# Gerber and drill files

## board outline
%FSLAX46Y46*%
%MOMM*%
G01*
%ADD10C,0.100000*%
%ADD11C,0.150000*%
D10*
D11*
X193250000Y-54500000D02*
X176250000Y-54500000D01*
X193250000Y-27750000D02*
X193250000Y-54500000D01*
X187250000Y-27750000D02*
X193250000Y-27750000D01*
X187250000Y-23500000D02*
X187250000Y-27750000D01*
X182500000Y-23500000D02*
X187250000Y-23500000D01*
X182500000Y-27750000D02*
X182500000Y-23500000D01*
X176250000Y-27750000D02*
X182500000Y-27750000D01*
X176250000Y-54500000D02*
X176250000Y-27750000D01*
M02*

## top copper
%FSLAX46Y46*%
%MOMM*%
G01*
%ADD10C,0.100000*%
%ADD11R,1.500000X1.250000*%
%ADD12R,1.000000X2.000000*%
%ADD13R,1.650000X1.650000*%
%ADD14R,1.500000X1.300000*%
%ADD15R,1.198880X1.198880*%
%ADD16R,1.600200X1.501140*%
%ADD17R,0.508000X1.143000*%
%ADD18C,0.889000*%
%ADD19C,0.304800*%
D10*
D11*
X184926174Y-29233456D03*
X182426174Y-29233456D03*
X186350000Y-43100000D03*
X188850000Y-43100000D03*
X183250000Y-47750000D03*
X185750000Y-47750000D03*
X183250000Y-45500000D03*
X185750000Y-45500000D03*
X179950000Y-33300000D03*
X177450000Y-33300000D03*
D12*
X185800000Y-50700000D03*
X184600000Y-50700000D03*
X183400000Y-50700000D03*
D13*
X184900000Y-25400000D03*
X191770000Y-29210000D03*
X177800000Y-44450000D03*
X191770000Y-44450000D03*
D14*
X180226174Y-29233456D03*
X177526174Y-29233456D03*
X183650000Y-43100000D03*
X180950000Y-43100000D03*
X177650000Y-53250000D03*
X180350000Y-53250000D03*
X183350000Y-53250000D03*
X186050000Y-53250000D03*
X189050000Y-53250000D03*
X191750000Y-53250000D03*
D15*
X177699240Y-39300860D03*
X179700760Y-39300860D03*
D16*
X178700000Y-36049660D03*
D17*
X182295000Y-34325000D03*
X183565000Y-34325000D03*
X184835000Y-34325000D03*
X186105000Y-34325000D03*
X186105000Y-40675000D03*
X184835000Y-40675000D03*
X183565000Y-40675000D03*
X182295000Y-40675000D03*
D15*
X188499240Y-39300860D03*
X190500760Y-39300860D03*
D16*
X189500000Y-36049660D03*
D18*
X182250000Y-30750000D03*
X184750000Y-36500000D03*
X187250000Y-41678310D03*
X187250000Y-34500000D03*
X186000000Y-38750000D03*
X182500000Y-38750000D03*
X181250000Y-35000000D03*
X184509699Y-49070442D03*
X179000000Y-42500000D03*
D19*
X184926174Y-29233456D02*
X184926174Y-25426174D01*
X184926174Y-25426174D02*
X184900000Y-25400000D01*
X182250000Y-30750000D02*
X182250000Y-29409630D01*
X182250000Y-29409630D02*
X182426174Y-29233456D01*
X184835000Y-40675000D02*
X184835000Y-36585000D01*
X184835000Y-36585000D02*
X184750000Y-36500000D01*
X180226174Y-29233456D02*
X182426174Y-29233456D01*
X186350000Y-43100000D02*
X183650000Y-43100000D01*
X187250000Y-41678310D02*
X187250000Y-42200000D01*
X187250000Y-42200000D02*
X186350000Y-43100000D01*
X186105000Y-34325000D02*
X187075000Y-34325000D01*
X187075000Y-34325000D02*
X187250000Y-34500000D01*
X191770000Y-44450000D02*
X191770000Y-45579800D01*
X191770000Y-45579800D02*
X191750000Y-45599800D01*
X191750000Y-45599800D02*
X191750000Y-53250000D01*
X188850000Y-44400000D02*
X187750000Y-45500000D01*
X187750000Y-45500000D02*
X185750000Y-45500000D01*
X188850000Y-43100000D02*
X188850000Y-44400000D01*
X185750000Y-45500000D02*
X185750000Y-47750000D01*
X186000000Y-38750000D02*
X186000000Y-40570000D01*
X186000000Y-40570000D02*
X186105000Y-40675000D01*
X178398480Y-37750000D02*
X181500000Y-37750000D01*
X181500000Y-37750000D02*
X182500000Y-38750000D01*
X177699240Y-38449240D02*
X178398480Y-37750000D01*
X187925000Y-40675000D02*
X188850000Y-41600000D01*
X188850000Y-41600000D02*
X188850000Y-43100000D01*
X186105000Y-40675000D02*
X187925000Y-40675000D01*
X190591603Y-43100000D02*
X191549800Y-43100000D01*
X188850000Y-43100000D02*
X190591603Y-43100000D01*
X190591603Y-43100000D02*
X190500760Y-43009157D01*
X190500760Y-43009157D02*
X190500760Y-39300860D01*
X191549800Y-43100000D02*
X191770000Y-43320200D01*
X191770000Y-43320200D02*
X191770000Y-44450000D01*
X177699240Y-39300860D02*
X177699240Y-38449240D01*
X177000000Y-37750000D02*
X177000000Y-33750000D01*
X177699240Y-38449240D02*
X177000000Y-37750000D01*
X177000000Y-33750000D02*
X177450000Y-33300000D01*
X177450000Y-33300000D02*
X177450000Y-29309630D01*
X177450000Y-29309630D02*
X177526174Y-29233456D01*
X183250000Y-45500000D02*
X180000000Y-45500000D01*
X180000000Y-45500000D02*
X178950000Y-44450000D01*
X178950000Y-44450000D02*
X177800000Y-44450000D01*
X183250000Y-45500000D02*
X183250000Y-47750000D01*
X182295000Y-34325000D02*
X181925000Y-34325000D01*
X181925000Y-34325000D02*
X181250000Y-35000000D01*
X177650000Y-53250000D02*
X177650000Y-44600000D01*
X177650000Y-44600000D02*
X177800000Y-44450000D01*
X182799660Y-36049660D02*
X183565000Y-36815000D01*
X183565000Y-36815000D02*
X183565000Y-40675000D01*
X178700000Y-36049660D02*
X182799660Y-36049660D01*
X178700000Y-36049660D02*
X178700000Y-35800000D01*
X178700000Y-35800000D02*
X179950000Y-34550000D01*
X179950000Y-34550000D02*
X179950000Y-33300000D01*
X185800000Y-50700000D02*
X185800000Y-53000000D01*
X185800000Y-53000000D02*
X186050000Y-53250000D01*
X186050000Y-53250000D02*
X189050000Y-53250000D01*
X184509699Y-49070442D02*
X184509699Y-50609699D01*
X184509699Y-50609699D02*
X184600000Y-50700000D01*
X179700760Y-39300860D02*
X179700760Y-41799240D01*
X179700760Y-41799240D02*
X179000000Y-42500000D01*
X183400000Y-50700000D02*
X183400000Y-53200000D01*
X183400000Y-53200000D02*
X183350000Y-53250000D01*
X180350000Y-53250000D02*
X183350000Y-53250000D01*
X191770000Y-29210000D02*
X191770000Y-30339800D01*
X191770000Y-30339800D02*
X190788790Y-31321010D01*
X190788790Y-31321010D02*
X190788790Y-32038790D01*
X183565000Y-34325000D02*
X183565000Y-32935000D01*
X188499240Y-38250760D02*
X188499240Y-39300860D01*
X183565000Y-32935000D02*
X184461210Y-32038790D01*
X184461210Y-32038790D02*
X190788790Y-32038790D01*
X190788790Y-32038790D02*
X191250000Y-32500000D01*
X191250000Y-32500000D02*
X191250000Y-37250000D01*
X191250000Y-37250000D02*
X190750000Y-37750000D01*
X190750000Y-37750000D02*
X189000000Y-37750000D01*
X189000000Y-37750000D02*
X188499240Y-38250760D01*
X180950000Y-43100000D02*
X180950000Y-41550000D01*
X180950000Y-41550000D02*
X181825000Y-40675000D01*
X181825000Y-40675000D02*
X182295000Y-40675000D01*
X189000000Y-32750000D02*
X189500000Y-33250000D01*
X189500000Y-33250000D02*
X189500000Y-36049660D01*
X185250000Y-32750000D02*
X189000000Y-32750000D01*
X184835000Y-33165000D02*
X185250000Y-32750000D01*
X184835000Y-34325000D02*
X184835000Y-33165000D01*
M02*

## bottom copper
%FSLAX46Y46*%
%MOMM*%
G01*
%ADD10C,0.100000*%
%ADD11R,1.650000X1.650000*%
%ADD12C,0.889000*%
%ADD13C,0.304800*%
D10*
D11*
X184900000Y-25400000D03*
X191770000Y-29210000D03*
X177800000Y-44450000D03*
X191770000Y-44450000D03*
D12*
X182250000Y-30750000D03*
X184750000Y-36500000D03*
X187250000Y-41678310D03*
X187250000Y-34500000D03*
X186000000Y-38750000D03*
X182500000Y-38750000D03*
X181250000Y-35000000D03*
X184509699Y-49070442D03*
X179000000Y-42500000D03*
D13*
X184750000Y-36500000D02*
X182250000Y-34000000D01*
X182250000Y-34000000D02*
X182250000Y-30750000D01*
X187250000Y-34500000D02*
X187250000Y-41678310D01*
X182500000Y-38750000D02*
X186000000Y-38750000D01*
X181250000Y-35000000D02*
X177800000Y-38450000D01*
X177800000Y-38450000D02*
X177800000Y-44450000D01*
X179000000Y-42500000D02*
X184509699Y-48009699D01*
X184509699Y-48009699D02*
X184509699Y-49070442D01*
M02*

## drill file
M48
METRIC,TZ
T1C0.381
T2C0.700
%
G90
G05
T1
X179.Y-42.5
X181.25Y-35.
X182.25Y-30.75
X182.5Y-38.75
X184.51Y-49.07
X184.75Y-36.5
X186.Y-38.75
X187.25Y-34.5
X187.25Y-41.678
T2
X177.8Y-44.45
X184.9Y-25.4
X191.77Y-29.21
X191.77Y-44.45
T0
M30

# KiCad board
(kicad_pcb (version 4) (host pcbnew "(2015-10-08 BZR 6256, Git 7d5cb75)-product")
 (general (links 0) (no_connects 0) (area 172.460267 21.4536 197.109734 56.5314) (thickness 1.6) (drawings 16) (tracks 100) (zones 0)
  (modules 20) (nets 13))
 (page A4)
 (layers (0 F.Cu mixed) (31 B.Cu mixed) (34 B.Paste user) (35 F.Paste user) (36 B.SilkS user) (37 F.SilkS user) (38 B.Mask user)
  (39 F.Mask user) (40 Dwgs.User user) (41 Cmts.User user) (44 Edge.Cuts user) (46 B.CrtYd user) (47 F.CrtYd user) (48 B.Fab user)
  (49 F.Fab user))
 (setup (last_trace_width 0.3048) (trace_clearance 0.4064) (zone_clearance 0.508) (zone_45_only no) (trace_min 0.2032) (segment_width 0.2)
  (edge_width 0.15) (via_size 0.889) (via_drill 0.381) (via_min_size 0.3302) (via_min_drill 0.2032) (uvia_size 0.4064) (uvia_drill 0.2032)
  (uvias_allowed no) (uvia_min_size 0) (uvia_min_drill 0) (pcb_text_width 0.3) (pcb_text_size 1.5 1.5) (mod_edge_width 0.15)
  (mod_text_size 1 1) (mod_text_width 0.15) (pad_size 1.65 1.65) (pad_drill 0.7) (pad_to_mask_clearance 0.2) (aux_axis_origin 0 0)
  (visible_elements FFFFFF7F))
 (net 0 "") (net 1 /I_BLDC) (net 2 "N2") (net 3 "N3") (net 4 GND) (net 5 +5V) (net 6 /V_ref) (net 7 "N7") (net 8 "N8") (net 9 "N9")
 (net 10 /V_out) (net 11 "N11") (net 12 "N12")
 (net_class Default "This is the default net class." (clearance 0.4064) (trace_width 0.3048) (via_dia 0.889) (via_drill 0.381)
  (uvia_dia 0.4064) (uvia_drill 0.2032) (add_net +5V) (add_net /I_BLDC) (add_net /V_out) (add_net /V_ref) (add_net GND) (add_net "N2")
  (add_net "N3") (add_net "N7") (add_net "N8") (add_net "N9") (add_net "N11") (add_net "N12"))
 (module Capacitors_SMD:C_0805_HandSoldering (layer F.Cu) (at 183.676174 29.233456 180)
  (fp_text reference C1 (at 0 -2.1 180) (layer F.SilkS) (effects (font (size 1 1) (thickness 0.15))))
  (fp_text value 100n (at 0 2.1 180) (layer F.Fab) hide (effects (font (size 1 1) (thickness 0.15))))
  (pad 1 smd rect (at -1.25 0 180) (size 1.5 1.25) (layers F.Cu F.Paste F.Mask) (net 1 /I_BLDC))
  (pad 2 smd rect (at 1.25 0 180) (size 1.5 1.25) (layers F.Cu F.Paste F.Mask) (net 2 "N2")))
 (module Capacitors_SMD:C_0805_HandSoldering (layer F.Cu) (at 187.6 43.1)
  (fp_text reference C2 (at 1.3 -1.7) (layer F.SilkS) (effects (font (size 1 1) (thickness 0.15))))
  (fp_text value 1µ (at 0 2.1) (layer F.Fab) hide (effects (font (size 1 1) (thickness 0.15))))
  (pad 1 smd rect (at -1.25 0) (size 1.5 1.25) (layers F.Cu F.Paste F.Mask) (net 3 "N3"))
  (pad 2 smd rect (at 1.25 0) (size 1.5 1.25) (layers F.Cu F.Paste F.Mask) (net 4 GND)))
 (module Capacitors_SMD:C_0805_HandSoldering (layer F.Cu) (at 184.5 47.75)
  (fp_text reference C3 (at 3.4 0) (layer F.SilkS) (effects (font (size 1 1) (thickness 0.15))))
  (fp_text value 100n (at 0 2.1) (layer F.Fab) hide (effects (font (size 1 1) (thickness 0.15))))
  (pad 1 smd rect (at -1.25 0) (size 1.5 1.25) (layers F.Cu F.Paste F.Mask) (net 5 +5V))
  (pad 2 smd rect (at 1.25 0) (size 1.5 1.25) (layers F.Cu F.Paste F.Mask) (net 4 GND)))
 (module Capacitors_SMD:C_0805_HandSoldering (layer F.Cu) (at 184.5 45.5)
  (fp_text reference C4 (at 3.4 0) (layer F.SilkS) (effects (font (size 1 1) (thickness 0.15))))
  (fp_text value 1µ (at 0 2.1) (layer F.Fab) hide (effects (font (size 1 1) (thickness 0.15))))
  (pad 1 smd rect (at -1.25 0) (size 1.5 1.25) (layers F.Cu F.Paste F.Mask) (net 5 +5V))
  (pad 2 smd rect (at 1.25 0) (size 1.5 1.25) (layers F.Cu F.Paste F.Mask) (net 4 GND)))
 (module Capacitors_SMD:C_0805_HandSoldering (layer F.Cu) (at 178.7 33.3 180)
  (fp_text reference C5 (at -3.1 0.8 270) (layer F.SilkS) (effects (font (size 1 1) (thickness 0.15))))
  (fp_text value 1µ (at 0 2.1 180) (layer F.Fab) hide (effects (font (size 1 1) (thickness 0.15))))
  (pad 1 smd rect (at -1.25 0 180) (size 1.5 1.25) (layers F.Cu F.Paste F.Mask) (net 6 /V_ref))
  (pad 2 smd rect (at 1.25 0 180) (size 1.5 1.25) (layers F.Cu F.Paste F.Mask) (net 4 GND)))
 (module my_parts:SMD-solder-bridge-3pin (layer F.Cu) (at 184.6 50.7 180) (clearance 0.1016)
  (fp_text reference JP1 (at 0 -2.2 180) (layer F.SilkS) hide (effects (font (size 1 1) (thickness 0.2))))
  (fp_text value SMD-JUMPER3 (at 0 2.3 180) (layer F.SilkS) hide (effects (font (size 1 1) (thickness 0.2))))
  (pad 1 smd rect (at -1.2 0 180) (size 1 2) (layers F.Cu F.Mask) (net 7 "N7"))
  (pad 2 smd rect (at 0 0 180) (size 1 2) (layers F.Cu F.Mask) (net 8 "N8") (solder_mask_margin 0.3))
  (pad 3 smd rect (at 1.2 0 180) (size 1 2) (layers F.Cu F.Mask) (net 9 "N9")))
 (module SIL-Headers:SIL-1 (layer F.Cu) (at 184.9 25.4)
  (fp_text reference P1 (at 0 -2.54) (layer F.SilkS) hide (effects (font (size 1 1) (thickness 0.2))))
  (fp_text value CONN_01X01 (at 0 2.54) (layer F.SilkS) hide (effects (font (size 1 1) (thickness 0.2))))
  (pad 1 thru_hole rect (at 0 0) (size 1.65 1.65) (drill 0.7) (layers *.Cu *.Mask) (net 1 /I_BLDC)))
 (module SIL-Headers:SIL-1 (layer F.Cu) (at 191.77 29.21)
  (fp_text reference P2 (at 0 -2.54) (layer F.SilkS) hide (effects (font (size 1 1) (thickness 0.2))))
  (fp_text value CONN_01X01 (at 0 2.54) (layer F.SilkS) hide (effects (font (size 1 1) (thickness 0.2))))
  (pad 1 thru_hole rect (at 0 0) (size 1.65 1.65) (drill 0.7) (layers *.Cu *.Mask) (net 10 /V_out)))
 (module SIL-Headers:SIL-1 (layer F.Cu) (at 177.8 44.45)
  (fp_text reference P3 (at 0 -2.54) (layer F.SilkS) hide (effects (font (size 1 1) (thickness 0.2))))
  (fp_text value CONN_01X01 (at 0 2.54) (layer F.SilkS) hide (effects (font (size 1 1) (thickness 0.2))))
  (pad 1 thru_hole rect (at 0 0) (size 1.65 1.65) (drill 0.7) (layers *.Cu *.Mask) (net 5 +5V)))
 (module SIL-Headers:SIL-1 (layer F.Cu) (at 191.77 44.45)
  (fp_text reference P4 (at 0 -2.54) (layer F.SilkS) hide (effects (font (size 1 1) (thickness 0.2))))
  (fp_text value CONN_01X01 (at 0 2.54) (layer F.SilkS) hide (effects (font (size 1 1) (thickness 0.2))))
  (pad 1 thru_hole rect (at 0 0) (size 1.65 1.65) (drill 0.7) (layers *.Cu *.Mask) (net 4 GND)))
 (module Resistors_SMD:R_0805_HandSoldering (layer F.Cu) (at 178.876174 29.233456 180)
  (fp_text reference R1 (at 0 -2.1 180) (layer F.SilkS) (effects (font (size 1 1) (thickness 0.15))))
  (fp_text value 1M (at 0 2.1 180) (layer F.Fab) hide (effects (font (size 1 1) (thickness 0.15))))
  (pad 1 smd rect (at -1.35 0 180) (size 1.5 1.3) (layers F.Cu F.Paste F.Mask) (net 2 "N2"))
  (pad 2 smd rect (at 1.35 0 180) (size 1.5 1.3) (layers F.Cu F.Paste F.Mask) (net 4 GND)))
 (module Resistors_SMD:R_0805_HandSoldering (layer F.Cu) (at 182.3 43.1 180)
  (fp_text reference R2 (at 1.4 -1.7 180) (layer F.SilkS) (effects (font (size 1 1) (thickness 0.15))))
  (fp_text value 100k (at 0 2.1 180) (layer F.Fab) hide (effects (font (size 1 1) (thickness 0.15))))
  (pad 1 smd rect (at -1.35 0 180) (size 1.5 1.3) (layers F.Cu F.Paste F.Mask) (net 3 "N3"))
  (pad 2 smd rect (at 1.35 0 180) (size 1.5 1.3) (layers F.Cu F.Paste F.Mask) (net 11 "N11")))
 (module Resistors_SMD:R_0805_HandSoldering (layer F.Cu) (at 179 53.25)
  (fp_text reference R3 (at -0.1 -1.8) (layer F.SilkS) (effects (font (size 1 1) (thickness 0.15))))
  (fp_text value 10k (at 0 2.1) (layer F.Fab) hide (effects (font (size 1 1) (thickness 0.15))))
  (pad 1 smd rect (at -1.35 0) (size 1.5 1.3) (layers F.Cu F.Paste F.Mask) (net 5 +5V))
  (pad 2 smd rect (at 1.35 0) (size 1.5 1.3) (layers F.Cu F.Paste F.Mask) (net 9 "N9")))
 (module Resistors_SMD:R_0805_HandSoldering (layer F.Cu) (at 184.7 53.25)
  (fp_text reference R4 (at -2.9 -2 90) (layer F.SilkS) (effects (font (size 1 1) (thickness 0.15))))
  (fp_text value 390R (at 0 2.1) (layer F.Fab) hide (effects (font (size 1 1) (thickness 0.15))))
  (pad 1 smd rect (at -1.35 0) (size 1.5 1.3) (layers F.Cu F.Paste F.Mask) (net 9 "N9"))
  (pad 2 smd rect (at 1.35 0) (size 1.5 1.3) (layers F.Cu F.Paste F.Mask) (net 7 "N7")))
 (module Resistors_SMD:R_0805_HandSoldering (layer F.Cu) (at 190.4 53.25)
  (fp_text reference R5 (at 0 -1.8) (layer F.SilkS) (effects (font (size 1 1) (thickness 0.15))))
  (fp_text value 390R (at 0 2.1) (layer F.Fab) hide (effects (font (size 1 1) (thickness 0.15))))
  (pad 1 smd rect (at -1.35 0) (size 1.5 1.3) (layers F.Cu F.Paste F.Mask) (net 7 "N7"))
  (pad 2 smd rect (at 1.35 0) (size 1.5 1.3) (layers F.Cu F.Paste F.Mask) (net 4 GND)))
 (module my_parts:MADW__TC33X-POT (layer F.Cu) (at 178.7 37.5)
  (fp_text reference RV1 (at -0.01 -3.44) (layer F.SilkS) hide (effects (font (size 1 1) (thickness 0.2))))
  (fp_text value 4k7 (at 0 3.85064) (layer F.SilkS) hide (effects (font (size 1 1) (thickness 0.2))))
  (pad 1 smd rect (at -1.00076 1.80086) (size 1.19888 1.19888) (layers F.Cu F.Paste F.Mask) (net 4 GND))
  (pad 3 smd rect (at 1.00076 1.80086) (size 1.19888 1.19888) (layers F.Cu F.Paste F.Mask) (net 8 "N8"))
  (pad 2 smd rect (at 0 -1.45034) (size 1.6002 1.50114) (layers F.Cu F.Paste F.Mask) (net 6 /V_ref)))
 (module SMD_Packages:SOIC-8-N (layer F.Cu) (at 184.2 37.5)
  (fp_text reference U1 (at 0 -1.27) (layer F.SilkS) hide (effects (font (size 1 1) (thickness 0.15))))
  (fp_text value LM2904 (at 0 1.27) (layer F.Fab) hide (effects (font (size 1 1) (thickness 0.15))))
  (pad 8 smd rect (at -1.905 -3.175) (size 0.508 1.143) (layers F.Cu F.Paste F.Mask) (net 5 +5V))
  (pad 7 smd rect (at -0.635 -3.175) (size 0.508 1.143) (layers F.Cu F.Paste F.Mask) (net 10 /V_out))
  (pad 6 smd rect (at 0.635 -3.175) (size 0.508 1.143) (layers F.Cu F.Paste F.Mask) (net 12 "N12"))
  (pad 5 smd rect (at 1.905 -3.175) (size 0.508 1.143) (layers F.Cu F.Paste F.Mask) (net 3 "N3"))
  (pad 4 smd rect (at 1.905 3.175) (size 0.508 1.143) (layers F.Cu F.Paste F.Mask) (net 4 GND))
  (pad 3 smd rect (at 0.635 3.175) (size 0.508 1.143) (layers F.Cu F.Paste F.Mask) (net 2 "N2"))
  (pad 2 smd rect (at -0.635 3.175) (size 0.508 1.143) (layers F.Cu F.Paste F.Mask) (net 6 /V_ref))
  (pad 1 smd rect (at -1.905 3.175) (size 0.508 1.143) (layers F.Cu F.Paste F.Mask) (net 11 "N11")))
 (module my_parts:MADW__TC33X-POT (layer F.Cu) (at 189.5 37.5)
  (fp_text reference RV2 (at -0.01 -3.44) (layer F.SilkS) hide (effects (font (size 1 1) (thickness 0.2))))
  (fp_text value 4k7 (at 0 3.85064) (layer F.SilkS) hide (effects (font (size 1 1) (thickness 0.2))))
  (pad 1 smd rect (at -1.00076 1.80086) (size 1.19888 1.19888) (layers F.Cu F.Paste F.Mask) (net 10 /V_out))
  (pad 3 smd rect (at 1.00076 1.80086) (size 1.19888 1.19888) (layers F.Cu F.Paste F.Mask) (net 4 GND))
  (pad 2 smd rect (at 0 -1.45034) (size 1.6002 1.50114) (layers F.Cu F.Paste F.Mask) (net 12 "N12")))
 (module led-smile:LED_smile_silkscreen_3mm (layer F.Cu) (at 180.25 48.5)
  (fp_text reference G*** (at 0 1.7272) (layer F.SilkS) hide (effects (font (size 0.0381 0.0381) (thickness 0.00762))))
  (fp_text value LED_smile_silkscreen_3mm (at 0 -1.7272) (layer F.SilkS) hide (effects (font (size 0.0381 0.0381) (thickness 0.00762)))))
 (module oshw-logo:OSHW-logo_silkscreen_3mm (layer F.Cu) (at 190.5 49)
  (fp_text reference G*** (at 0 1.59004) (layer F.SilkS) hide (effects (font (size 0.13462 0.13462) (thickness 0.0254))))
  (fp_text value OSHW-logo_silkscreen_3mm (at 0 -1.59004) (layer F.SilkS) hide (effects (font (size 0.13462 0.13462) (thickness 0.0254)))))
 (gr_line (start 193.25 54.5) (end 176.25 54.5) (layer Edge.Cuts) (width 0.15))
 (gr_line (start 193.25 27.75) (end 193.25 54.5) (layer Edge.Cuts) (width 0.15))
 (gr_line (start 187.25 27.75) (end 193.25 27.75) (layer Edge.Cuts) (width 0.15))
 (gr_line (start 187.25 23.5) (end 187.25 27.75) (layer Edge.Cuts) (width 0.15))
 (gr_line (start 182.5 23.5) (end 187.25 23.5) (layer Edge.Cuts) (width 0.15))
 (gr_line (start 182.5 27.75) (end 182.5 23.5) (layer Edge.Cuts) (width 0.15))
 (gr_line (start 176.25 27.75) (end 182.5 27.75) (layer Edge.Cuts) (width 0.15))
 (gr_line (start 176.25 54.5) (end 176.25 27.75) (layer Edge.Cuts) (width 0.15))
 (segment (start 184.926174 29.233456) (end 184.926174 25.426174) (width 0.3048) (layer F.Cu) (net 1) (status 30))
 (segment (start 184.926174 25.426174) (end 184.9 25.4) (width 0.3048) (layer F.Cu) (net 1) (status 30))
 (segment (start 182.25 30.75) (end 182.25 29.40963) (width 0.3048) (layer F.Cu) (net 2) (status 20))
 (segment (start 182.25 29.40963) (end 182.426174 29.233456) (width 0.3048) (layer F.Cu) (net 2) (status 30))
 (segment (start 184.75 36.5) (end 182.25 34) (width 0.3048) (layer B.Cu) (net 2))
 (segment (start 182.25 34) (end 182.25 30.75) (width 0.3048) (layer B.Cu) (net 2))
 (via (at 182.25 30.75) (size 0.889) (drill 0.381) (layers F.Cu B.Cu) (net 2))
 (segment (start 184.835 40.675) (end 184.835 36.585) (width 0.3048) (layer F.Cu) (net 2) (status 10))
 (segment (start 184.835 36.585) (end 184.75 36.5) (width 0.3048) (layer F.Cu) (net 2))
 (via (at 184.75 36.5) (size 0.889) (drill 0.381) (layers F.Cu B.Cu) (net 2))
 (segment (start 180.226174 29.233456) (end 182.426174 29.233456) (width 0.3048) (layer F.Cu) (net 2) (status 30))
 (segment (start 186.35 43.1) (end 183.65 43.1) (width 0.3048) (layer F.Cu) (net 3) (status 30))
 (segment (start 187.25 41.67831) (end 187.25 42.2) (width 0.3048) (layer F.Cu) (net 3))
 (segment (start 187.25 42.2) (end 186.35 43.1) (width 0.3048) (layer F.Cu) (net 3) (status 20))
 (segment (start 187.25 34.5) (end 187.25 41.67831) (width 0.3048) (layer B.Cu) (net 3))
 (via (at 187.25 41.67831) (size 0.889) (drill 0.381) (layers F.Cu B.Cu) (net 3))
 (segment (start 186.105 34.325) (end 187.075 34.325) (width 0.3048) (layer F.Cu) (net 3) (status 10))
 (segment (start 187.075 34.325) (end 187.25 34.5) (width 0.3048) (layer F.Cu) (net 3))
 (via (at 187.25 34.5) (size 0.889) (drill 0.381) (layers F.Cu B.Cu) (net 3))
 (segment (start 191.77 44.45) (end 191.77 45.5798) (width 0.3048) (layer F.Cu) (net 4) (status 10))
 (segment (start 191.77 45.5798) (end 191.75 45.5998) (width 0.3048) (layer F.Cu) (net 4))
 (segment (start 191.75 45.5998) (end 191.75 53.25) (width 0.3048) (layer F.Cu) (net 4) (status 20))
 (segment (start 188.85 44.4) (end 187.75 45.5) (width 0.3048) (layer F.Cu) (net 4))
 (segment (start 187.75 45.5) (end 185.75 45.5) (width 0.3048) (layer F.Cu) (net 4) (status 20))
 (segment (start 188.85 43.1) (end 188.85 44.4) (width 0.3048) (layer F.Cu) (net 4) (status 10))
 (segment (start 185.75 45.5) (end 185.75 47.75) (width 0.3048) (layer F.Cu) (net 4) (status 30))
 (segment (start 186 38.75) (end 186 40.57) (width 0.3048) (layer F.Cu) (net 4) (status 20))
 (segment (start 186 40.57) (end 186.105 40.675) (width 0.3048) (layer F.Cu) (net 4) (status 30))
 (segment (start 182.5 38.75) (end 186 38.75) (width 0.3048) (layer B.Cu) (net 4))
 (via (at 186 38.75) (size 0.889) (drill 0.381) (layers F.Cu B.Cu) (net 4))
 (segment (start 178.39848 37.75) (end 181.5 37.75) (width 0.3048) (layer F.Cu) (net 4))
 (segment (start 181.5 37.75) (end 182.5 38.75) (width 0.3048) (layer F.Cu) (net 4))
 (segment (start 177.69924 38.44924) (end 178.39848 37.75) (width 0.3048) (layer F.Cu) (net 4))
 (via (at 182.5 38.75) (size 0.889) (drill 0.381) (layers F.Cu B.Cu) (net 4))
 (segment (start 187.925 40.675) (end 188.85 41.6) (width 0.3048) (layer F.Cu) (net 4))
 (segment (start 188.85 41.6) (end 188.85 43.1) (width 0.3048) (layer F.Cu) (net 4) (status 20))
 (segment (start 186.105 40.675) (end 187.925 40.675) (width 0.3048) (layer F.Cu) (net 4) (status 10))
 (segment (start 190.591603 43.1) (end 191.5498 43.1) (width 0.3048) (layer F.Cu) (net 4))
 (segment (start 188.85 43.1) (end 190.591603 43.1) (width 0.3048) (layer F.Cu) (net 4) (status 10))
 (segment (start 190.591603 43.1) (end 190.50076 43.009157) (width 0.3048) (layer F.Cu) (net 4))
 (segment (start 190.50076 43.009157) (end 190.50076 39.30086) (width 0.3048) (layer F.Cu) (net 4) (status 20))
 (segment (start 191.5498 43.1) (end 191.77 43.3202) (width 0.3048) (layer F.Cu) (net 4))
 (segment (start 191.77 43.3202) (end 191.77 44.45) (width 0.3048) (layer F.Cu) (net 4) (status 20))
 (segment (start 177.69924 39.30086) (end 177.69924 38.44924) (width 0.3048) (layer F.Cu) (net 4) (status 10))
 (segment (start 177 37.75) (end 177 33.75) (width 0.3048) (layer F.Cu) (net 4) (status 20))
 (segment (start 177.69924 38.44924) (end 177 37.75) (width 0.3048) (layer F.Cu) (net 4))
 (segment (start 177 33.75) (end 177.45 33.3) (width 0.3048) (layer F.Cu) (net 4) (status 30))
 (segment (start 177.45 33.3) (end 177.45 29.30963) (width 0.3048) (layer F.Cu) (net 4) (status 30))
 (segment (start 177.45 29.30963) (end 177.526174 29.233456) (width 0.3048) (layer F.Cu) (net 4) (status 30))
 (segment (start 183.25 45.5) (end 180 45.5) (width 0.3048) (layer F.Cu) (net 5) (status 10))
 (segment (start 180 45.5) (end 178.95 44.45) (width 0.3048) (layer F.Cu) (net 5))
 (segment (start 178.95 44.45) (end 177.8 44.45) (width 0.3048) (layer F.Cu) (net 5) (status 20))
 (segment (start 183.25 45.5) (end 183.25 47.75) (width 0.3048) (layer F.Cu) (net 5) (status 30))
 (segment (start 181.25 35) (end 177.8 38.45) (width 0.3048) (layer B.Cu) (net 5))
 (segment (start 177.8 38.45) (end 177.8 44.45) (width 0.3048) (layer B.Cu) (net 5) (status 20))
 (segment (start 182.295 34.325) (end 181.925 34.325) (width 0.3048) (layer F.Cu) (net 5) (status 10))
 (via (at 181.25 35) (size 0.889) (drill 0.381) (layers F.Cu B.Cu) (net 5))
 (segment (start 181.925 34.325) (end 181.25 35) (width 0.3048) (layer F.Cu) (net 5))
 (segment (start 177.65 53.25) (end 177.65 44.6) (width 0.3048) (layer F.Cu) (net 5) (status 30))
 (segment (start 177.65 44.6) (end 177.8 44.45) (width 0.3048) (layer F.Cu) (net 5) (status 30))
 (segment (start 182.79966 36.04966) (end 183.565 36.815) (width 0.3048) (layer F.Cu) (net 6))
 (segment (start 183.565 36.815) (end 183.565 40.675) (width 0.3048) (layer F.Cu) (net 6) (status 20))
 (segment (start 178.7 36.04966) (end 182.79966 36.04966) (width 0.3048) (layer F.Cu) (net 6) (status 10))
 (segment (start 178.7 36.04966) (end 178.7 35.8) (width 0.3048) (layer F.Cu) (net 6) (status 30))
 (segment (start 178.7 35.8) (end 179.95 34.55) (width 0.3048) (layer F.Cu) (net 6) (status 10))
 (segment (start 179.95 34.55) (end 179.95 33.3) (width 0.3048) (layer F.Cu) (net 6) (status 20))
 (segment (start 185.8 50.7) (end 185.8 53) (width 0.3048) (layer F.Cu) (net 7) (status 30))
 (segment (start 185.8 53) (end 186.05 53.25) (width 0.3048) (layer F.Cu) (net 7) (status 30))
 (segment (start 186.05 53.25) (end 189.05 53.25) (width 0.3048) (layer F.Cu) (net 7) (status 30))
 (segment (start 184.509699 49.070442) (end 184.509699 50.609699) (width 0.3048) (layer F.Cu) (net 8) (status 20))
 (segment (start 184.509699 50.609699) (end 184.6 50.7) (width 0.3048) (layer F.Cu) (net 8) (status 30))
 (segment (start 179 42.5) (end 184.509699 48.009699) (width 0.3048) (layer B.Cu) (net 8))
 (segment (start 184.509699 48.009699) (end 184.509699 49.070442) (width 0.3048) (layer B.Cu) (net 8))
 (via (at 184.509699 49.070442) (size 0.889) (drill 0.381) (layers F.Cu B.Cu) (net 8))
 (segment (start 179.70076 39.30086) (end 179.70076 41.79924) (width 0.3048) (layer F.Cu) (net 8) (status 10))
 (segment (start 179.70076 41.79924) (end 179 42.5) (width 0.3048) (layer F.Cu) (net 8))
 (via (at 179 42.5) (size 0.889) (drill 0.381) (layers F.Cu B.Cu) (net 8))
 (segment (start 183.4 50.7) (end 183.4 53.2) (width 0.3048) (layer F.Cu) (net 9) (status 30))
 (segment (start 183.4 53.2) (end 183.35 53.25) (width 0.3048) (layer F.Cu) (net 9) (status 30))
 (segment (start 180.35 53.25) (end 183.35 53.25) (width 0.3048) (layer F.Cu) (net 9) (status 30))
 (segment (start 191.77 29.21) (end 191.77 30.3398) (width 0.3048) (layer F.Cu) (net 10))
 (segment (start 191.77 30.3398) (end 190.78879 31.32101) (width 0.3048) (layer F.Cu) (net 10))
 (segment (start 190.78879 31.32101) (end 190.78879 32.03879) (width 0.3048) (layer F.Cu) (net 10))
 (segment (start 183.565 34.325) (end 183.565 32.935) (width 0.3048) (layer F.Cu) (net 10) (status 10))
 (segment (start 188.49924 38.25076) (end 188.49924 39.30086) (width 0.3048) (layer F.Cu) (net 10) (status 20))
 (segment (start 183.565 32.935) (end 184.46121 32.03879) (width 0.3048) (layer F.Cu) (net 10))
 (segment (start 184.46121 32.03879) (end 190.78879 32.03879) (width 0.3048) (layer F.Cu) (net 10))
 (segment (start 190.78879 32.03879) (end 191.25 32.5) (width 0.3048) (layer F.Cu) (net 10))
 (segment (start 191.25 32.5) (end 191.25 37.25) (width 0.3048) (layer F.Cu) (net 10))
 (segment (start 191.25 37.25) (end 190.75 37.75) (width 0.3048) (layer F.Cu) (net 10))
 (segment (start 190.75 37.75) (end 189 37.75) (width 0.3048) (layer F.Cu) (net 10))
 (segment (start 189 37.75) (end 188.49924 38.25076) (width 0.3048) (layer F.Cu) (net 10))
 (segment (start 180.95 43.1) (end 180.95 41.55) (width 0.3048) (layer F.Cu) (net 11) (status 10))
 (segment (start 180.95 41.55) (end 181.825 40.675) (width 0.3048) (layer F.Cu) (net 11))
 (segment (start 181.825 40.675) (end 182.295 40.675) (width 0.3048) (layer F.Cu) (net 11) (status 20))
 (segment (start 189 32.75) (end 189.5 33.25) (width 0.3048) (layer F.Cu) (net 12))
 (segment (start 189.5 33.25) (end 189.5 36.04966) (width 0.3048) (layer F.Cu) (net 12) (status 20))
 (segment (start 185.25 32.75) (end 189 32.75) (width 0.3048) (layer F.Cu) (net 12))
 (segment (start 184.835 33.165) (end 185.25 32.75) (width 0.3048) (layer F.Cu) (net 12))
 (segment (start 184.835 34.325) (end 184.835 33.165) (width 0.3048) (layer F.Cu) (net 12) (status 10)))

